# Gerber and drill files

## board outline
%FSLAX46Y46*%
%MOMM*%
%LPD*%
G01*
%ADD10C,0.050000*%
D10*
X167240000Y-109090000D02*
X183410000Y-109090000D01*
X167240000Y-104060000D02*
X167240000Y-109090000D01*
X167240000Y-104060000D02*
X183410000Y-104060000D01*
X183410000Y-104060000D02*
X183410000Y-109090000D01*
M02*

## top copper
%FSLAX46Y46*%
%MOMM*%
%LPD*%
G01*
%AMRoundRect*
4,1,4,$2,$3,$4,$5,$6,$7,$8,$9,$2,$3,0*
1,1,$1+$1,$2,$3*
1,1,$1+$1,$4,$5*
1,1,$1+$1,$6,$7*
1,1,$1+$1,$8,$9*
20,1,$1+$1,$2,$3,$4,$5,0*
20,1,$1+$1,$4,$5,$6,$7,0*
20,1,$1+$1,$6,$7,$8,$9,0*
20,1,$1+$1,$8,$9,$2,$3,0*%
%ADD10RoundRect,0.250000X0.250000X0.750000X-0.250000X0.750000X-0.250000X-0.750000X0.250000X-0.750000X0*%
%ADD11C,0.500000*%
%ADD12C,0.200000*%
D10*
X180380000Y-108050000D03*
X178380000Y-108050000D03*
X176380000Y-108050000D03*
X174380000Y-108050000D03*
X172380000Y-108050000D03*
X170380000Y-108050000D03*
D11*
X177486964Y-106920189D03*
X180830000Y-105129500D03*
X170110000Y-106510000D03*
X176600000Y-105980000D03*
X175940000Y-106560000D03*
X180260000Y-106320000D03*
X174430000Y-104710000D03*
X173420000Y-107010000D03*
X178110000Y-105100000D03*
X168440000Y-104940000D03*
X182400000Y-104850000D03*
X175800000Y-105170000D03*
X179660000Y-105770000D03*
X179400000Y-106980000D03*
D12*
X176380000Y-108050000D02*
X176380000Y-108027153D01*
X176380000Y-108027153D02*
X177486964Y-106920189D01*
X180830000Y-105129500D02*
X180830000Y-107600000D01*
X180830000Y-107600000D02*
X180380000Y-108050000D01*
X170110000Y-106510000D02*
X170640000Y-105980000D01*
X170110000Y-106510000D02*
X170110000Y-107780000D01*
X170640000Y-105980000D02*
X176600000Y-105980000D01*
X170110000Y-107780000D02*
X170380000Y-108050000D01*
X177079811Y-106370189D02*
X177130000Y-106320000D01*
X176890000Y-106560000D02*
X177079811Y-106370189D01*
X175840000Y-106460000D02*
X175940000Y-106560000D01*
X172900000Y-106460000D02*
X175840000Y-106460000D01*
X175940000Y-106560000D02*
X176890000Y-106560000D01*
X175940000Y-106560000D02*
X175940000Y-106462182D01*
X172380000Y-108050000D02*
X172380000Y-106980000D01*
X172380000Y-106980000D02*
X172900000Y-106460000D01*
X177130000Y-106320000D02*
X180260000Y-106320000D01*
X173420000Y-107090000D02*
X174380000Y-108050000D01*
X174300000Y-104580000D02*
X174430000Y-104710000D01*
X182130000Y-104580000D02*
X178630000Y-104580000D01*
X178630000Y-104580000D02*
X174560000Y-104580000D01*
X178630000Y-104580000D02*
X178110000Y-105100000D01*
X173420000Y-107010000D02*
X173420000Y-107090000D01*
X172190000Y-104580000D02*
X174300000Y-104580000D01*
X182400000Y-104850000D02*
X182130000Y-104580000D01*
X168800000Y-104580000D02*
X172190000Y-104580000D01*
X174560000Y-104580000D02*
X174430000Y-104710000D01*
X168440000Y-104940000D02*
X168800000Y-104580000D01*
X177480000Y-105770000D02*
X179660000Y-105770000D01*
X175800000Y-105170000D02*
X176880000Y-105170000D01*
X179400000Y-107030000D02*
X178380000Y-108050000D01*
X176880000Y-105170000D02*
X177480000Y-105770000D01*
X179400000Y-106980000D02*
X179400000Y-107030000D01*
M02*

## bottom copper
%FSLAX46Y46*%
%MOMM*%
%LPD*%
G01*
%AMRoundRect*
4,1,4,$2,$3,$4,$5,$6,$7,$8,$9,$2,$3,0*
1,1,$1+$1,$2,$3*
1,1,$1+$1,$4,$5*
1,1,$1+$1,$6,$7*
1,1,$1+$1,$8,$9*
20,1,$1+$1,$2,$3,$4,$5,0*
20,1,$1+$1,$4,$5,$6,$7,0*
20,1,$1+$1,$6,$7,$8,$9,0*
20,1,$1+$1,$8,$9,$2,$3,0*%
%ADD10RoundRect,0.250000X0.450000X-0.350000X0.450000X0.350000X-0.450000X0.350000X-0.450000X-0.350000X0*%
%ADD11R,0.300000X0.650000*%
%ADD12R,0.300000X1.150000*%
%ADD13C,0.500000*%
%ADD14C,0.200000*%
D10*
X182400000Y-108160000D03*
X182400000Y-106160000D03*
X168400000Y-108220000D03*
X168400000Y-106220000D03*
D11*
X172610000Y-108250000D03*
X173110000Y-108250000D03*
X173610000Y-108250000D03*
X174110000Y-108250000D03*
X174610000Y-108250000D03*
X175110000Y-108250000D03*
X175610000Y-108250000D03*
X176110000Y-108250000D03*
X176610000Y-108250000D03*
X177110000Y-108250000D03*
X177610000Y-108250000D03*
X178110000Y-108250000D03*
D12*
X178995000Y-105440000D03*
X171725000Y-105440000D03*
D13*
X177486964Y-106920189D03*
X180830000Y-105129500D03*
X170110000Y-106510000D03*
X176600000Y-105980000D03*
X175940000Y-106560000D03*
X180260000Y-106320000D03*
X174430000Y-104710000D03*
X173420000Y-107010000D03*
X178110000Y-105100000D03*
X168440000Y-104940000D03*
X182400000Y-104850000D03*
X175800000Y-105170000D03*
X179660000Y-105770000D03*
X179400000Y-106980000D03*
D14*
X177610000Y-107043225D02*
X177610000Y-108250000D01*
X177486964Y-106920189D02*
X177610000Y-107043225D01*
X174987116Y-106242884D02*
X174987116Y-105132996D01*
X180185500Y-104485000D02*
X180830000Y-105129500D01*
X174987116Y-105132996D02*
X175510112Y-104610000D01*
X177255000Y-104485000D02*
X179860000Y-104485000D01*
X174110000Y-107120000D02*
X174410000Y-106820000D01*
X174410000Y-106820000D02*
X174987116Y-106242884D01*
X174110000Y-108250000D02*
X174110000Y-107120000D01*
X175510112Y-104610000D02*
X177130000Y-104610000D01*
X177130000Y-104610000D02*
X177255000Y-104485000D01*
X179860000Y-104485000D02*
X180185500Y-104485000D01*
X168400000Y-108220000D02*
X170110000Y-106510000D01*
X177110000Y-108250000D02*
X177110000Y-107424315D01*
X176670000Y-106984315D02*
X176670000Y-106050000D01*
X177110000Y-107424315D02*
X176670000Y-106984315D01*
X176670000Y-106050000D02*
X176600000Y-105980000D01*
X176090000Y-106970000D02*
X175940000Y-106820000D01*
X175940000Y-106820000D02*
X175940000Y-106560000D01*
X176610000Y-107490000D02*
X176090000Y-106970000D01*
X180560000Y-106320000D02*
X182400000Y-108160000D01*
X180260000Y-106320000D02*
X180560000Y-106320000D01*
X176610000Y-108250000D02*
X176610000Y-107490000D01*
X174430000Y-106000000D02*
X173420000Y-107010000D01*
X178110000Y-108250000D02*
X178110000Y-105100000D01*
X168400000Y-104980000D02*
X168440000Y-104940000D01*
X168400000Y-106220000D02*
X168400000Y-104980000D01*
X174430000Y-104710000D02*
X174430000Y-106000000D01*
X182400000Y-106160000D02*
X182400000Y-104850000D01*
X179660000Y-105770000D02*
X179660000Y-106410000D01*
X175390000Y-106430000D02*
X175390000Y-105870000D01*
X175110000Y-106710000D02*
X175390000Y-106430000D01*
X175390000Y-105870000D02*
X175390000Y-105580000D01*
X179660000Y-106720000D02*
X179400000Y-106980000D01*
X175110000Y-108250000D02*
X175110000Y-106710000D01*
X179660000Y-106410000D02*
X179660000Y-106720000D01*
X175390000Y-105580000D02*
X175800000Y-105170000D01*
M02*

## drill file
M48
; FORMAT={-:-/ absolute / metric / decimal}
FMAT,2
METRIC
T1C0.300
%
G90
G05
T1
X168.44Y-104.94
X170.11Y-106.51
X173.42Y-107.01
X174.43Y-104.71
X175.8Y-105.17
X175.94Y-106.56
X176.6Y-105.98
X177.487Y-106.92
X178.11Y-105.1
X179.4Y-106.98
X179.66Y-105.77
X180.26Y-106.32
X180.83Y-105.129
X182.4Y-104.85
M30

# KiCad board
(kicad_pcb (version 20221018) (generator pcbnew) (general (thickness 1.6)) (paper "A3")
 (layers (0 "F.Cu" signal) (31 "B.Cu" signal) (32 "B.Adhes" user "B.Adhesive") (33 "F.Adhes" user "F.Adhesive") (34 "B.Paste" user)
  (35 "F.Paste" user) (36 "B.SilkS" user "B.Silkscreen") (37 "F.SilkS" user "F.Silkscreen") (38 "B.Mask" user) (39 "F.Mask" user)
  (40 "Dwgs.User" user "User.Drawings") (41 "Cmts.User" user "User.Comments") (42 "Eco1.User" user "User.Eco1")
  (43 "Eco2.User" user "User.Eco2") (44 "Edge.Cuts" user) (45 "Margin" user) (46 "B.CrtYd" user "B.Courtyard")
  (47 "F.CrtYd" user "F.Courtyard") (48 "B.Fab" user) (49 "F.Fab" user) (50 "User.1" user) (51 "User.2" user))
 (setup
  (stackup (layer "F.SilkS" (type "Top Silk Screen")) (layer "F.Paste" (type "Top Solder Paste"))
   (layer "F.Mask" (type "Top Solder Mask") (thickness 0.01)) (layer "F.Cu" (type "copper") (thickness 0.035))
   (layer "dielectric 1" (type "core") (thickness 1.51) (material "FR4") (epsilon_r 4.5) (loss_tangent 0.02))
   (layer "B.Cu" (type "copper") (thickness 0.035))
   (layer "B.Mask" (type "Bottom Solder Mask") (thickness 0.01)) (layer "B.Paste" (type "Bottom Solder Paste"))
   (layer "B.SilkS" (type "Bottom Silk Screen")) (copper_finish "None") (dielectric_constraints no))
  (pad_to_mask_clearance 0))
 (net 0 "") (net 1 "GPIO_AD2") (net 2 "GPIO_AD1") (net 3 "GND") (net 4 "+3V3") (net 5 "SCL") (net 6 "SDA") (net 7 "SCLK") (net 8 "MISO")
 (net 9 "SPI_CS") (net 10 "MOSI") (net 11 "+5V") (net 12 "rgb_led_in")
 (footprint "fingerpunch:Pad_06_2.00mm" (layer "F.Cu") (at 175.38 108.05 180)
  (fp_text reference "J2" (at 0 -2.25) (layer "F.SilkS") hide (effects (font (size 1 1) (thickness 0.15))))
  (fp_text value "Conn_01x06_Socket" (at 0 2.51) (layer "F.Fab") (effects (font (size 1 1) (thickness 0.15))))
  (pad "1" smd roundrect (at -5 0 180) (size 1 2) (layers "F.Cu" "F.Paste" "F.Mask") (roundrect_rratio 0.25) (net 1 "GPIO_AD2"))
  (pad "2" smd roundrect (at -3 0 180) (size 1 2) (layers "F.Cu" "F.Paste" "F.Mask") (roundrect_rratio 0.25) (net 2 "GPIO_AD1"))
  (pad "3" smd roundrect (at -1 0 180) (size 1 2) (layers "F.Cu" "F.Paste" "F.Mask") (roundrect_rratio 0.25) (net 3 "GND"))
  (pad "4" smd roundrect (at 1 0 180) (size 1 2) (layers "F.Cu" "F.Paste" "F.Mask") (roundrect_rratio 0.25) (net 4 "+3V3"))
  (pad "5" smd roundrect (at 3 0 180) (size 1 2) (layers "F.Cu" "F.Paste" "F.Mask") (roundrect_rratio 0.25) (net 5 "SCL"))
  (pad "6" smd roundrect (at 5 0 180) (size 1 2) (layers "F.Cu" "F.Paste" "F.Mask") (roundrect_rratio 0.25) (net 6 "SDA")))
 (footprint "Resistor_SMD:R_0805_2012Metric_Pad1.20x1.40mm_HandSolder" (layer "B.Cu") (at 182.4 107.16 90)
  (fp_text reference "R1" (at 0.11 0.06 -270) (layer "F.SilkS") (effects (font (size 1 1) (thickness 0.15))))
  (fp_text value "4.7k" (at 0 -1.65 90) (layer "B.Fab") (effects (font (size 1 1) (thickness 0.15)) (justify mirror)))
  (pad "1" smd roundrect (at -1 0 90) (size 1.2 1.4) (layers "B.Cu" "B.Paste" "B.Mask") (roundrect_rratio 0.2083333333) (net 5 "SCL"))
  (pad "2" smd roundrect (at 1 0 90) (size 1.2 1.4) (layers "B.Cu" "B.Paste" "B.Mask") (roundrect_rratio 0.2083333333) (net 4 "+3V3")))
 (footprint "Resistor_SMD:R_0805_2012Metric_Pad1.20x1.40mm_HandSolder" (layer "B.Cu") (at 168.4 107.22 90)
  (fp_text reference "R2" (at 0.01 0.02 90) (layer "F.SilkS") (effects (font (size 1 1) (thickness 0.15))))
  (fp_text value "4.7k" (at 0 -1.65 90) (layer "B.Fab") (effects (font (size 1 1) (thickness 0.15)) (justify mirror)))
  (pad "1" smd roundrect (at -1 0 90) (size 1.2 1.4) (layers "B.Cu" "B.Paste" "B.Mask") (roundrect_rratio 0.2083333333) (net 6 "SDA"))
  (pad "2" smd roundrect (at 1 0 90) (size 1.2 1.4) (layers "B.Cu" "B.Paste" "B.Mask") (roundrect_rratio 0.2083333333) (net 4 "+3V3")))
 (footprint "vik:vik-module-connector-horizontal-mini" (layer "B.Cu") (at 175.36 106.14)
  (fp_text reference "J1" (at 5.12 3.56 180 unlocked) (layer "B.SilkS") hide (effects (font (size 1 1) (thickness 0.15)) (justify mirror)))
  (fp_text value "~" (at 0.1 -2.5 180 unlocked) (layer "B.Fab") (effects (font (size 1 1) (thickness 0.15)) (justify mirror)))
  (pad "1" smd rect (at -2.75 2.11) (size 0.3 0.65) (layers "B.Cu" "B.Paste" "B.Mask") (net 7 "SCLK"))
  (pad "2" smd rect (at -2.25 2.11) (size 0.3 0.65) (layers "B.Cu" "B.Paste" "B.Mask") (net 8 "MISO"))
  (pad "3" smd rect (at -1.75 2.11) (size 0.3 0.65) (layers "B.Cu" "B.Paste" "B.Mask") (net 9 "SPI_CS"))
  (pad "4" smd rect (at -1.25 2.11) (size 0.3 0.65) (layers "B.Cu" "B.Paste" "B.Mask") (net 1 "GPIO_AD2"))
  (pad "5" smd rect (at -0.75 2.11) (size 0.3 0.65) (layers "B.Cu" "B.Paste" "B.Mask") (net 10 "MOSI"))
  (pad "6" smd rect (at -0.25 2.11) (size 0.3 0.65) (layers "B.Cu" "B.Paste" "B.Mask") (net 2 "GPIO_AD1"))
  (pad "7" smd rect (at 0.25 2.11) (size 0.3 0.65) (layers "B.Cu" "B.Paste" "B.Mask") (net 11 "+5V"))
  (pad "8" smd rect (at 0.75 2.11) (size 0.3 0.65) (layers "B.Cu" "B.Paste" "B.Mask") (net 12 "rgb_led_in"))
  (pad "9" smd rect (at 1.25 2.11) (size 0.3 0.65) (layers "B.Cu" "B.Paste" "B.Mask") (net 5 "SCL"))
  (pad "10" smd rect (at 1.75 2.11) (size 0.3 0.65) (layers "B.Cu" "B.Paste" "B.Mask") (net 6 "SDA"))
  (pad "11" smd rect (at 2.25 2.11) (size 0.3 0.65) (layers "B.Cu" "B.Paste" "B.Mask") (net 3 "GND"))
  (pad "12" smd rect (at 2.75 2.11) (size 0.3 0.65) (layers "B.Cu" "B.Paste" "B.Mask") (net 4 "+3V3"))
  (pad "13" smd rect (at 3.635 -0.7) (size 0.3 1.15) (layers "B.Cu" "B.Paste" "B.Mask"))
  (pad "14" smd rect (at -3.635 -0.7) (size 0.3 1.15) (layers "B.Cu" "B.Paste" "B.Mask")))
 (gr_line (start 167.24 109.09) (end 183.41 109.09) (stroke (width 0.05) (type default)) (layer "Edge.Cuts"))
 (gr_line (start 167.24 104.06) (end 167.24 109.09) (stroke (width 0.05) (type default)) (layer "Edge.Cuts"))
 (gr_line (start 167.24 104.06) (end 183.41 104.06) (stroke (width 0.05) (type default)) (layer "Edge.Cuts"))
 (gr_line (start 183.41 104.06) (end 183.41 109.09) (stroke (width 0.05) (type default)) (layer "Edge.Cuts"))
 (segment (start 176.38 108.05) (end 176.38 108.027153) (width 0.2) (layer "F.Cu") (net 3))
 (segment (start 176.38 108.027153) (end 177.486964 106.920189) (width 0.2) (layer "F.Cu") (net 3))
 (via (at 177.486964 106.920189) (size 0.5) (drill 0.3) (layers "F.Cu" "B.Cu") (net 3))
 (segment (start 177.61 107.043225) (end 177.61 108.25) (width 0.2) (layer "B.Cu") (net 3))
 (segment (start 177.486964 106.920189) (end 177.61 107.043225) (width 0.2) (layer "B.Cu") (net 3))
 (segment (start 180.83 105.1295) (end 180.83 107.6) (width 0.2) (layer "F.Cu") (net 1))
 (segment (start 180.83 107.6) (end 180.38 108.05) (width 0.2) (layer "F.Cu") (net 1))
 (via (at 180.83 105.1295) (size 0.5) (drill 0.3) (layers "F.Cu" "B.Cu") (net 1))
 (segment (start 174.987116 106.242884) (end 174.987116 105.132996) (width 0.2) (layer "B.Cu") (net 1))
 (segment (start 180.1855 104.485) (end 180.83 105.1295) (width 0.2) (layer "B.Cu") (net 1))
 (segment (start 174.987116 105.132996) (end 175.510112 104.61) (width 0.2) (layer "B.Cu") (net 1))
 (segment (start 177.255 104.485) (end 179.86 104.485) (width 0.2) (layer "B.Cu") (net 1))
 (segment (start 174.11 107.12) (end 174.41 106.82) (width 0.2) (layer "B.Cu") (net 1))
 (segment (start 174.41 106.82) (end 174.987116 106.242884) (width 0.2) (layer "B.Cu") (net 1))
 (segment (start 174.11 108.25) (end 174.11 107.12) (width 0.2) (layer "B.Cu") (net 1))
 (segment (start 175.510112 104.61) (end 177.13 104.61) (width 0.2) (layer "B.Cu") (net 1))
 (segment (start 177.13 104.61) (end 177.255 104.485) (width 0.2) (layer "B.Cu") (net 1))
 (segment (start 179.86 104.485) (end 180.1855 104.485) (width 0.2) (layer "B.Cu") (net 1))
 (segment (start 170.11 106.51) (end 170.64 105.98) (width 0.2) (layer "F.Cu") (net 6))
 (segment (start 170.11 106.51) (end 170.11 107.78) (width 0.2) (layer "F.Cu") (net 6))
 (segment (start 170.64 105.98) (end 176.6 105.98) (width 0.2) (layer "F.Cu") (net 6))
 (segment (start 170.11 107.78) (end 170.38 108.05) (width 0.2) (layer "F.Cu") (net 6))
 (via (at 170.11 106.51) (size 0.5) (drill 0.3) (layers "F.Cu" "B.Cu") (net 6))
 (via (at 176.6 105.98) (size 0.5) (drill 0.3) (layers "F.Cu" "B.Cu") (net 6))
 (segment (start 168.4 108.22) (end 170.11 106.51) (width 0.2) (layer "B.Cu") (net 6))
 (segment (start 177.11 108.25) (end 177.11 107.424315) (width 0.2) (layer "B.Cu") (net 6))
 (segment (start 176.67 106.984315) (end 176.67 106.05) (width 0.2) (layer "B.Cu") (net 6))
 (segment (start 177.11 107.424315) (end 176.67 106.984315) (width 0.2) (layer "B.Cu") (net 6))
 (segment (start 176.67 106.05) (end 176.6 105.98) (width 0.2) (layer "B.Cu") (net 6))
 (segment (start 177.079811 106.370189) (end 177.13 106.32) (width 0.2) (layer "F.Cu") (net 5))
 (segment (start 176.89 106.56) (end 177.079811 106.370189) (width 0.2) (layer "F.Cu") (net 5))
 (segment (start 175.84 106.46) (end 175.94 106.56) (width 0.2) (layer "F.Cu") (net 5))
 (segment (start 172.9 106.46) (end 175.84 106.46) (width 0.2) (layer "F.Cu") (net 5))
 (segment (start 175.94 106.56) (end 176.89 106.56) (width 0.2) (layer "F.Cu") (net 5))
 (segment (start 175.94 106.56) (end 175.94 106.462182) (width 0.2) (layer "F.Cu") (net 5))
 (segment (start 172.38 108.05) (end 172.38 106.98) (width 0.2) (layer "F.Cu") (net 5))
 (segment (start 172.38 106.98) (end 172.9 106.46) (width 0.2) (layer "F.Cu") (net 5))
 (segment (start 177.13 106.32) (end 180.26 106.32) (width 0.2) (layer "F.Cu") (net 5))
 (via (at 175.94 106.56) (size 0.5) (drill 0.3) (layers "F.Cu" "B.Cu") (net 5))
 (via (at 180.26 106.32) (size 0.5) (drill 0.3) (layers "F.Cu" "B.Cu") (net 5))
 (segment (start 176.09 106.97) (end 175.94 106.82) (width 0.2) (layer "B.Cu") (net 5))
 (segment (start 175.94 106.82) (end 175.94 106.56) (width 0.2) (layer "B.Cu") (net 5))
 (segment (start 176.61 107.49) (end 176.09 106.97) (width 0.2) (layer "B.Cu") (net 5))
 (segment (start 180.56 106.32) (end 182.4 108.16) (width 0.2) (layer "B.Cu") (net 5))
 (segment (start 180.26 106.32) (end 180.56 106.32) (width 0.2) (layer "B.Cu") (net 5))
 (segment (start 176.61 108.25) (end 176.61 107.49) (width 0.2) (layer "B.Cu") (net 5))
 (segment (start 173.42 107.09) (end 174.38 108.05) (width 0.2) (layer "F.Cu") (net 4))
 (segment (start 174.3 104.58) (end 174.43 104.71) (width 0.2) (layer "F.Cu") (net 4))
 (segment (start 182.13 104.58) (end 178.63 104.58) (width 0.2) (layer "F.Cu") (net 4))
 (segment (start 178.63 104.58) (end 174.56 104.58) (width 0.2) (layer "F.Cu") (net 4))
 (segment (start 178.63 104.58) (end 178.11 105.1) (width 0.2) (layer "F.Cu") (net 4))
 (segment (start 173.42 107.01) (end 173.42 107.09) (width 0.2) (layer "F.Cu") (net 4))
 (segment (start 172.19 104.58) (end 174.3 104.58) (width 0.2) (layer "F.Cu") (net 4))
 (segment (start 182.4 104.85) (end 182.13 104.58) (width 0.2) (layer "F.Cu") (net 4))
 (segment (start 168.8 104.58) (end 172.19 104.58) (width 0.2) (layer "F.Cu") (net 4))
 (segment (start 174.56 104.58) (end 174.43 104.71) (width 0.2) (layer "F.Cu") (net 4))
 (segment (start 168.44 104.94) (end 168.8 104.58) (width 0.2) (layer "F.Cu") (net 4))
 (via (at 174.43 104.71) (size 0.5) (drill 0.3) (layers "F.Cu" "B.Cu") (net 4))
 (via (at 173.42 107.01) (size 0.5) (drill 0.3) (layers "F.Cu" "B.Cu") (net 4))
 (via (at 178.11 105.1) (size 0.5) (drill 0.3) (layers "F.Cu" "B.Cu") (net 4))
 (via (at 168.44 104.94) (size 0.5) (drill 0.3) (layers "F.Cu" "B.Cu") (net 4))
 (via (at 182.4 104.85) (size 0.5) (drill 0.3) (layers "F.Cu" "B.Cu") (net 4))
 (segment (start 174.43 106) (end 173.42 107.01) (width 0.2) (layer "B.Cu") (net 4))
 (segment (start 178.11 108.25) (end 178.11 105.1) (width 0.2) (layer "B.Cu") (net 4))
 (segment (start 168.4 104.98) (end 168.44 104.94) (width 0.2) (layer "B.Cu") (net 4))
 (segment (start 168.4 106.22) (end 168.4 104.98) (width 0.2) (layer "B.Cu") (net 4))
 (segment (start 174.43 104.71) (end 174.43 106) (width 0.2) (layer "B.Cu") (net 4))
 (segment (start 182.4 106.16) (end 182.4 104.85) (width 0.2) (layer "B.Cu") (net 4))
 (segment (start 177.48 105.77) (end 179.66 105.77) (width 0.2) (layer "F.Cu") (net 2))
 (segment (start 175.8 105.17) (end 176.88 105.17) (width 0.2) (layer "F.Cu") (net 2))
 (segment (start 179.4 107.03) (end 178.38 108.05) (width 0.2) (layer "F.Cu") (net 2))
 (segment (start 176.88 105.17) (end 177.48 105.77) (width 0.2) (layer "F.Cu") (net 2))
 (segment (start 179.4 106.98) (end 179.4 107.03) (width 0.2) (layer "F.Cu") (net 2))
 (via (at 175.8 105.17) (size 0.5) (drill 0.3) (layers "F.Cu" "B.Cu") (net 2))
 (via (at 179.66 105.77) (size 0.5) (drill 0.3) (layers "F.Cu" "B.Cu") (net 2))
 (via (at 179.4 106.98) (size 0.5) (drill 0.3) (layers "F.Cu" "B.Cu") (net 2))
 (segment (start 179.66 105.77) (end 179.66 106.41) (width 0.2) (layer "B.Cu") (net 2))
 (segment (start 175.39 106.43) (end 175.39 105.87) (width 0.2) (layer "B.Cu") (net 2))
 (segment (start 175.11 106.71) (end 175.39 106.43) (width 0.2) (layer "B.Cu") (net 2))
 (segment (start 175.39 105.87) (end 175.39 105.58) (width 0.2) (layer "B.Cu") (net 2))
 (segment (start 179.66 106.72) (end 179.4 106.98) (width 0.2) (layer "B.Cu") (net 2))
 (segment (start 175.11 108.25) (end 175.11 106.71) (width 0.2) (layer "B.Cu") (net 2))
 (segment (start 179.66 106.41) (end 179.66 106.72) (width 0.2) (layer "B.Cu") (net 2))
 (segment (start 175.39 105.58) (end 175.8 105.17) (width 0.2) (layer "B.Cu") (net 2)))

